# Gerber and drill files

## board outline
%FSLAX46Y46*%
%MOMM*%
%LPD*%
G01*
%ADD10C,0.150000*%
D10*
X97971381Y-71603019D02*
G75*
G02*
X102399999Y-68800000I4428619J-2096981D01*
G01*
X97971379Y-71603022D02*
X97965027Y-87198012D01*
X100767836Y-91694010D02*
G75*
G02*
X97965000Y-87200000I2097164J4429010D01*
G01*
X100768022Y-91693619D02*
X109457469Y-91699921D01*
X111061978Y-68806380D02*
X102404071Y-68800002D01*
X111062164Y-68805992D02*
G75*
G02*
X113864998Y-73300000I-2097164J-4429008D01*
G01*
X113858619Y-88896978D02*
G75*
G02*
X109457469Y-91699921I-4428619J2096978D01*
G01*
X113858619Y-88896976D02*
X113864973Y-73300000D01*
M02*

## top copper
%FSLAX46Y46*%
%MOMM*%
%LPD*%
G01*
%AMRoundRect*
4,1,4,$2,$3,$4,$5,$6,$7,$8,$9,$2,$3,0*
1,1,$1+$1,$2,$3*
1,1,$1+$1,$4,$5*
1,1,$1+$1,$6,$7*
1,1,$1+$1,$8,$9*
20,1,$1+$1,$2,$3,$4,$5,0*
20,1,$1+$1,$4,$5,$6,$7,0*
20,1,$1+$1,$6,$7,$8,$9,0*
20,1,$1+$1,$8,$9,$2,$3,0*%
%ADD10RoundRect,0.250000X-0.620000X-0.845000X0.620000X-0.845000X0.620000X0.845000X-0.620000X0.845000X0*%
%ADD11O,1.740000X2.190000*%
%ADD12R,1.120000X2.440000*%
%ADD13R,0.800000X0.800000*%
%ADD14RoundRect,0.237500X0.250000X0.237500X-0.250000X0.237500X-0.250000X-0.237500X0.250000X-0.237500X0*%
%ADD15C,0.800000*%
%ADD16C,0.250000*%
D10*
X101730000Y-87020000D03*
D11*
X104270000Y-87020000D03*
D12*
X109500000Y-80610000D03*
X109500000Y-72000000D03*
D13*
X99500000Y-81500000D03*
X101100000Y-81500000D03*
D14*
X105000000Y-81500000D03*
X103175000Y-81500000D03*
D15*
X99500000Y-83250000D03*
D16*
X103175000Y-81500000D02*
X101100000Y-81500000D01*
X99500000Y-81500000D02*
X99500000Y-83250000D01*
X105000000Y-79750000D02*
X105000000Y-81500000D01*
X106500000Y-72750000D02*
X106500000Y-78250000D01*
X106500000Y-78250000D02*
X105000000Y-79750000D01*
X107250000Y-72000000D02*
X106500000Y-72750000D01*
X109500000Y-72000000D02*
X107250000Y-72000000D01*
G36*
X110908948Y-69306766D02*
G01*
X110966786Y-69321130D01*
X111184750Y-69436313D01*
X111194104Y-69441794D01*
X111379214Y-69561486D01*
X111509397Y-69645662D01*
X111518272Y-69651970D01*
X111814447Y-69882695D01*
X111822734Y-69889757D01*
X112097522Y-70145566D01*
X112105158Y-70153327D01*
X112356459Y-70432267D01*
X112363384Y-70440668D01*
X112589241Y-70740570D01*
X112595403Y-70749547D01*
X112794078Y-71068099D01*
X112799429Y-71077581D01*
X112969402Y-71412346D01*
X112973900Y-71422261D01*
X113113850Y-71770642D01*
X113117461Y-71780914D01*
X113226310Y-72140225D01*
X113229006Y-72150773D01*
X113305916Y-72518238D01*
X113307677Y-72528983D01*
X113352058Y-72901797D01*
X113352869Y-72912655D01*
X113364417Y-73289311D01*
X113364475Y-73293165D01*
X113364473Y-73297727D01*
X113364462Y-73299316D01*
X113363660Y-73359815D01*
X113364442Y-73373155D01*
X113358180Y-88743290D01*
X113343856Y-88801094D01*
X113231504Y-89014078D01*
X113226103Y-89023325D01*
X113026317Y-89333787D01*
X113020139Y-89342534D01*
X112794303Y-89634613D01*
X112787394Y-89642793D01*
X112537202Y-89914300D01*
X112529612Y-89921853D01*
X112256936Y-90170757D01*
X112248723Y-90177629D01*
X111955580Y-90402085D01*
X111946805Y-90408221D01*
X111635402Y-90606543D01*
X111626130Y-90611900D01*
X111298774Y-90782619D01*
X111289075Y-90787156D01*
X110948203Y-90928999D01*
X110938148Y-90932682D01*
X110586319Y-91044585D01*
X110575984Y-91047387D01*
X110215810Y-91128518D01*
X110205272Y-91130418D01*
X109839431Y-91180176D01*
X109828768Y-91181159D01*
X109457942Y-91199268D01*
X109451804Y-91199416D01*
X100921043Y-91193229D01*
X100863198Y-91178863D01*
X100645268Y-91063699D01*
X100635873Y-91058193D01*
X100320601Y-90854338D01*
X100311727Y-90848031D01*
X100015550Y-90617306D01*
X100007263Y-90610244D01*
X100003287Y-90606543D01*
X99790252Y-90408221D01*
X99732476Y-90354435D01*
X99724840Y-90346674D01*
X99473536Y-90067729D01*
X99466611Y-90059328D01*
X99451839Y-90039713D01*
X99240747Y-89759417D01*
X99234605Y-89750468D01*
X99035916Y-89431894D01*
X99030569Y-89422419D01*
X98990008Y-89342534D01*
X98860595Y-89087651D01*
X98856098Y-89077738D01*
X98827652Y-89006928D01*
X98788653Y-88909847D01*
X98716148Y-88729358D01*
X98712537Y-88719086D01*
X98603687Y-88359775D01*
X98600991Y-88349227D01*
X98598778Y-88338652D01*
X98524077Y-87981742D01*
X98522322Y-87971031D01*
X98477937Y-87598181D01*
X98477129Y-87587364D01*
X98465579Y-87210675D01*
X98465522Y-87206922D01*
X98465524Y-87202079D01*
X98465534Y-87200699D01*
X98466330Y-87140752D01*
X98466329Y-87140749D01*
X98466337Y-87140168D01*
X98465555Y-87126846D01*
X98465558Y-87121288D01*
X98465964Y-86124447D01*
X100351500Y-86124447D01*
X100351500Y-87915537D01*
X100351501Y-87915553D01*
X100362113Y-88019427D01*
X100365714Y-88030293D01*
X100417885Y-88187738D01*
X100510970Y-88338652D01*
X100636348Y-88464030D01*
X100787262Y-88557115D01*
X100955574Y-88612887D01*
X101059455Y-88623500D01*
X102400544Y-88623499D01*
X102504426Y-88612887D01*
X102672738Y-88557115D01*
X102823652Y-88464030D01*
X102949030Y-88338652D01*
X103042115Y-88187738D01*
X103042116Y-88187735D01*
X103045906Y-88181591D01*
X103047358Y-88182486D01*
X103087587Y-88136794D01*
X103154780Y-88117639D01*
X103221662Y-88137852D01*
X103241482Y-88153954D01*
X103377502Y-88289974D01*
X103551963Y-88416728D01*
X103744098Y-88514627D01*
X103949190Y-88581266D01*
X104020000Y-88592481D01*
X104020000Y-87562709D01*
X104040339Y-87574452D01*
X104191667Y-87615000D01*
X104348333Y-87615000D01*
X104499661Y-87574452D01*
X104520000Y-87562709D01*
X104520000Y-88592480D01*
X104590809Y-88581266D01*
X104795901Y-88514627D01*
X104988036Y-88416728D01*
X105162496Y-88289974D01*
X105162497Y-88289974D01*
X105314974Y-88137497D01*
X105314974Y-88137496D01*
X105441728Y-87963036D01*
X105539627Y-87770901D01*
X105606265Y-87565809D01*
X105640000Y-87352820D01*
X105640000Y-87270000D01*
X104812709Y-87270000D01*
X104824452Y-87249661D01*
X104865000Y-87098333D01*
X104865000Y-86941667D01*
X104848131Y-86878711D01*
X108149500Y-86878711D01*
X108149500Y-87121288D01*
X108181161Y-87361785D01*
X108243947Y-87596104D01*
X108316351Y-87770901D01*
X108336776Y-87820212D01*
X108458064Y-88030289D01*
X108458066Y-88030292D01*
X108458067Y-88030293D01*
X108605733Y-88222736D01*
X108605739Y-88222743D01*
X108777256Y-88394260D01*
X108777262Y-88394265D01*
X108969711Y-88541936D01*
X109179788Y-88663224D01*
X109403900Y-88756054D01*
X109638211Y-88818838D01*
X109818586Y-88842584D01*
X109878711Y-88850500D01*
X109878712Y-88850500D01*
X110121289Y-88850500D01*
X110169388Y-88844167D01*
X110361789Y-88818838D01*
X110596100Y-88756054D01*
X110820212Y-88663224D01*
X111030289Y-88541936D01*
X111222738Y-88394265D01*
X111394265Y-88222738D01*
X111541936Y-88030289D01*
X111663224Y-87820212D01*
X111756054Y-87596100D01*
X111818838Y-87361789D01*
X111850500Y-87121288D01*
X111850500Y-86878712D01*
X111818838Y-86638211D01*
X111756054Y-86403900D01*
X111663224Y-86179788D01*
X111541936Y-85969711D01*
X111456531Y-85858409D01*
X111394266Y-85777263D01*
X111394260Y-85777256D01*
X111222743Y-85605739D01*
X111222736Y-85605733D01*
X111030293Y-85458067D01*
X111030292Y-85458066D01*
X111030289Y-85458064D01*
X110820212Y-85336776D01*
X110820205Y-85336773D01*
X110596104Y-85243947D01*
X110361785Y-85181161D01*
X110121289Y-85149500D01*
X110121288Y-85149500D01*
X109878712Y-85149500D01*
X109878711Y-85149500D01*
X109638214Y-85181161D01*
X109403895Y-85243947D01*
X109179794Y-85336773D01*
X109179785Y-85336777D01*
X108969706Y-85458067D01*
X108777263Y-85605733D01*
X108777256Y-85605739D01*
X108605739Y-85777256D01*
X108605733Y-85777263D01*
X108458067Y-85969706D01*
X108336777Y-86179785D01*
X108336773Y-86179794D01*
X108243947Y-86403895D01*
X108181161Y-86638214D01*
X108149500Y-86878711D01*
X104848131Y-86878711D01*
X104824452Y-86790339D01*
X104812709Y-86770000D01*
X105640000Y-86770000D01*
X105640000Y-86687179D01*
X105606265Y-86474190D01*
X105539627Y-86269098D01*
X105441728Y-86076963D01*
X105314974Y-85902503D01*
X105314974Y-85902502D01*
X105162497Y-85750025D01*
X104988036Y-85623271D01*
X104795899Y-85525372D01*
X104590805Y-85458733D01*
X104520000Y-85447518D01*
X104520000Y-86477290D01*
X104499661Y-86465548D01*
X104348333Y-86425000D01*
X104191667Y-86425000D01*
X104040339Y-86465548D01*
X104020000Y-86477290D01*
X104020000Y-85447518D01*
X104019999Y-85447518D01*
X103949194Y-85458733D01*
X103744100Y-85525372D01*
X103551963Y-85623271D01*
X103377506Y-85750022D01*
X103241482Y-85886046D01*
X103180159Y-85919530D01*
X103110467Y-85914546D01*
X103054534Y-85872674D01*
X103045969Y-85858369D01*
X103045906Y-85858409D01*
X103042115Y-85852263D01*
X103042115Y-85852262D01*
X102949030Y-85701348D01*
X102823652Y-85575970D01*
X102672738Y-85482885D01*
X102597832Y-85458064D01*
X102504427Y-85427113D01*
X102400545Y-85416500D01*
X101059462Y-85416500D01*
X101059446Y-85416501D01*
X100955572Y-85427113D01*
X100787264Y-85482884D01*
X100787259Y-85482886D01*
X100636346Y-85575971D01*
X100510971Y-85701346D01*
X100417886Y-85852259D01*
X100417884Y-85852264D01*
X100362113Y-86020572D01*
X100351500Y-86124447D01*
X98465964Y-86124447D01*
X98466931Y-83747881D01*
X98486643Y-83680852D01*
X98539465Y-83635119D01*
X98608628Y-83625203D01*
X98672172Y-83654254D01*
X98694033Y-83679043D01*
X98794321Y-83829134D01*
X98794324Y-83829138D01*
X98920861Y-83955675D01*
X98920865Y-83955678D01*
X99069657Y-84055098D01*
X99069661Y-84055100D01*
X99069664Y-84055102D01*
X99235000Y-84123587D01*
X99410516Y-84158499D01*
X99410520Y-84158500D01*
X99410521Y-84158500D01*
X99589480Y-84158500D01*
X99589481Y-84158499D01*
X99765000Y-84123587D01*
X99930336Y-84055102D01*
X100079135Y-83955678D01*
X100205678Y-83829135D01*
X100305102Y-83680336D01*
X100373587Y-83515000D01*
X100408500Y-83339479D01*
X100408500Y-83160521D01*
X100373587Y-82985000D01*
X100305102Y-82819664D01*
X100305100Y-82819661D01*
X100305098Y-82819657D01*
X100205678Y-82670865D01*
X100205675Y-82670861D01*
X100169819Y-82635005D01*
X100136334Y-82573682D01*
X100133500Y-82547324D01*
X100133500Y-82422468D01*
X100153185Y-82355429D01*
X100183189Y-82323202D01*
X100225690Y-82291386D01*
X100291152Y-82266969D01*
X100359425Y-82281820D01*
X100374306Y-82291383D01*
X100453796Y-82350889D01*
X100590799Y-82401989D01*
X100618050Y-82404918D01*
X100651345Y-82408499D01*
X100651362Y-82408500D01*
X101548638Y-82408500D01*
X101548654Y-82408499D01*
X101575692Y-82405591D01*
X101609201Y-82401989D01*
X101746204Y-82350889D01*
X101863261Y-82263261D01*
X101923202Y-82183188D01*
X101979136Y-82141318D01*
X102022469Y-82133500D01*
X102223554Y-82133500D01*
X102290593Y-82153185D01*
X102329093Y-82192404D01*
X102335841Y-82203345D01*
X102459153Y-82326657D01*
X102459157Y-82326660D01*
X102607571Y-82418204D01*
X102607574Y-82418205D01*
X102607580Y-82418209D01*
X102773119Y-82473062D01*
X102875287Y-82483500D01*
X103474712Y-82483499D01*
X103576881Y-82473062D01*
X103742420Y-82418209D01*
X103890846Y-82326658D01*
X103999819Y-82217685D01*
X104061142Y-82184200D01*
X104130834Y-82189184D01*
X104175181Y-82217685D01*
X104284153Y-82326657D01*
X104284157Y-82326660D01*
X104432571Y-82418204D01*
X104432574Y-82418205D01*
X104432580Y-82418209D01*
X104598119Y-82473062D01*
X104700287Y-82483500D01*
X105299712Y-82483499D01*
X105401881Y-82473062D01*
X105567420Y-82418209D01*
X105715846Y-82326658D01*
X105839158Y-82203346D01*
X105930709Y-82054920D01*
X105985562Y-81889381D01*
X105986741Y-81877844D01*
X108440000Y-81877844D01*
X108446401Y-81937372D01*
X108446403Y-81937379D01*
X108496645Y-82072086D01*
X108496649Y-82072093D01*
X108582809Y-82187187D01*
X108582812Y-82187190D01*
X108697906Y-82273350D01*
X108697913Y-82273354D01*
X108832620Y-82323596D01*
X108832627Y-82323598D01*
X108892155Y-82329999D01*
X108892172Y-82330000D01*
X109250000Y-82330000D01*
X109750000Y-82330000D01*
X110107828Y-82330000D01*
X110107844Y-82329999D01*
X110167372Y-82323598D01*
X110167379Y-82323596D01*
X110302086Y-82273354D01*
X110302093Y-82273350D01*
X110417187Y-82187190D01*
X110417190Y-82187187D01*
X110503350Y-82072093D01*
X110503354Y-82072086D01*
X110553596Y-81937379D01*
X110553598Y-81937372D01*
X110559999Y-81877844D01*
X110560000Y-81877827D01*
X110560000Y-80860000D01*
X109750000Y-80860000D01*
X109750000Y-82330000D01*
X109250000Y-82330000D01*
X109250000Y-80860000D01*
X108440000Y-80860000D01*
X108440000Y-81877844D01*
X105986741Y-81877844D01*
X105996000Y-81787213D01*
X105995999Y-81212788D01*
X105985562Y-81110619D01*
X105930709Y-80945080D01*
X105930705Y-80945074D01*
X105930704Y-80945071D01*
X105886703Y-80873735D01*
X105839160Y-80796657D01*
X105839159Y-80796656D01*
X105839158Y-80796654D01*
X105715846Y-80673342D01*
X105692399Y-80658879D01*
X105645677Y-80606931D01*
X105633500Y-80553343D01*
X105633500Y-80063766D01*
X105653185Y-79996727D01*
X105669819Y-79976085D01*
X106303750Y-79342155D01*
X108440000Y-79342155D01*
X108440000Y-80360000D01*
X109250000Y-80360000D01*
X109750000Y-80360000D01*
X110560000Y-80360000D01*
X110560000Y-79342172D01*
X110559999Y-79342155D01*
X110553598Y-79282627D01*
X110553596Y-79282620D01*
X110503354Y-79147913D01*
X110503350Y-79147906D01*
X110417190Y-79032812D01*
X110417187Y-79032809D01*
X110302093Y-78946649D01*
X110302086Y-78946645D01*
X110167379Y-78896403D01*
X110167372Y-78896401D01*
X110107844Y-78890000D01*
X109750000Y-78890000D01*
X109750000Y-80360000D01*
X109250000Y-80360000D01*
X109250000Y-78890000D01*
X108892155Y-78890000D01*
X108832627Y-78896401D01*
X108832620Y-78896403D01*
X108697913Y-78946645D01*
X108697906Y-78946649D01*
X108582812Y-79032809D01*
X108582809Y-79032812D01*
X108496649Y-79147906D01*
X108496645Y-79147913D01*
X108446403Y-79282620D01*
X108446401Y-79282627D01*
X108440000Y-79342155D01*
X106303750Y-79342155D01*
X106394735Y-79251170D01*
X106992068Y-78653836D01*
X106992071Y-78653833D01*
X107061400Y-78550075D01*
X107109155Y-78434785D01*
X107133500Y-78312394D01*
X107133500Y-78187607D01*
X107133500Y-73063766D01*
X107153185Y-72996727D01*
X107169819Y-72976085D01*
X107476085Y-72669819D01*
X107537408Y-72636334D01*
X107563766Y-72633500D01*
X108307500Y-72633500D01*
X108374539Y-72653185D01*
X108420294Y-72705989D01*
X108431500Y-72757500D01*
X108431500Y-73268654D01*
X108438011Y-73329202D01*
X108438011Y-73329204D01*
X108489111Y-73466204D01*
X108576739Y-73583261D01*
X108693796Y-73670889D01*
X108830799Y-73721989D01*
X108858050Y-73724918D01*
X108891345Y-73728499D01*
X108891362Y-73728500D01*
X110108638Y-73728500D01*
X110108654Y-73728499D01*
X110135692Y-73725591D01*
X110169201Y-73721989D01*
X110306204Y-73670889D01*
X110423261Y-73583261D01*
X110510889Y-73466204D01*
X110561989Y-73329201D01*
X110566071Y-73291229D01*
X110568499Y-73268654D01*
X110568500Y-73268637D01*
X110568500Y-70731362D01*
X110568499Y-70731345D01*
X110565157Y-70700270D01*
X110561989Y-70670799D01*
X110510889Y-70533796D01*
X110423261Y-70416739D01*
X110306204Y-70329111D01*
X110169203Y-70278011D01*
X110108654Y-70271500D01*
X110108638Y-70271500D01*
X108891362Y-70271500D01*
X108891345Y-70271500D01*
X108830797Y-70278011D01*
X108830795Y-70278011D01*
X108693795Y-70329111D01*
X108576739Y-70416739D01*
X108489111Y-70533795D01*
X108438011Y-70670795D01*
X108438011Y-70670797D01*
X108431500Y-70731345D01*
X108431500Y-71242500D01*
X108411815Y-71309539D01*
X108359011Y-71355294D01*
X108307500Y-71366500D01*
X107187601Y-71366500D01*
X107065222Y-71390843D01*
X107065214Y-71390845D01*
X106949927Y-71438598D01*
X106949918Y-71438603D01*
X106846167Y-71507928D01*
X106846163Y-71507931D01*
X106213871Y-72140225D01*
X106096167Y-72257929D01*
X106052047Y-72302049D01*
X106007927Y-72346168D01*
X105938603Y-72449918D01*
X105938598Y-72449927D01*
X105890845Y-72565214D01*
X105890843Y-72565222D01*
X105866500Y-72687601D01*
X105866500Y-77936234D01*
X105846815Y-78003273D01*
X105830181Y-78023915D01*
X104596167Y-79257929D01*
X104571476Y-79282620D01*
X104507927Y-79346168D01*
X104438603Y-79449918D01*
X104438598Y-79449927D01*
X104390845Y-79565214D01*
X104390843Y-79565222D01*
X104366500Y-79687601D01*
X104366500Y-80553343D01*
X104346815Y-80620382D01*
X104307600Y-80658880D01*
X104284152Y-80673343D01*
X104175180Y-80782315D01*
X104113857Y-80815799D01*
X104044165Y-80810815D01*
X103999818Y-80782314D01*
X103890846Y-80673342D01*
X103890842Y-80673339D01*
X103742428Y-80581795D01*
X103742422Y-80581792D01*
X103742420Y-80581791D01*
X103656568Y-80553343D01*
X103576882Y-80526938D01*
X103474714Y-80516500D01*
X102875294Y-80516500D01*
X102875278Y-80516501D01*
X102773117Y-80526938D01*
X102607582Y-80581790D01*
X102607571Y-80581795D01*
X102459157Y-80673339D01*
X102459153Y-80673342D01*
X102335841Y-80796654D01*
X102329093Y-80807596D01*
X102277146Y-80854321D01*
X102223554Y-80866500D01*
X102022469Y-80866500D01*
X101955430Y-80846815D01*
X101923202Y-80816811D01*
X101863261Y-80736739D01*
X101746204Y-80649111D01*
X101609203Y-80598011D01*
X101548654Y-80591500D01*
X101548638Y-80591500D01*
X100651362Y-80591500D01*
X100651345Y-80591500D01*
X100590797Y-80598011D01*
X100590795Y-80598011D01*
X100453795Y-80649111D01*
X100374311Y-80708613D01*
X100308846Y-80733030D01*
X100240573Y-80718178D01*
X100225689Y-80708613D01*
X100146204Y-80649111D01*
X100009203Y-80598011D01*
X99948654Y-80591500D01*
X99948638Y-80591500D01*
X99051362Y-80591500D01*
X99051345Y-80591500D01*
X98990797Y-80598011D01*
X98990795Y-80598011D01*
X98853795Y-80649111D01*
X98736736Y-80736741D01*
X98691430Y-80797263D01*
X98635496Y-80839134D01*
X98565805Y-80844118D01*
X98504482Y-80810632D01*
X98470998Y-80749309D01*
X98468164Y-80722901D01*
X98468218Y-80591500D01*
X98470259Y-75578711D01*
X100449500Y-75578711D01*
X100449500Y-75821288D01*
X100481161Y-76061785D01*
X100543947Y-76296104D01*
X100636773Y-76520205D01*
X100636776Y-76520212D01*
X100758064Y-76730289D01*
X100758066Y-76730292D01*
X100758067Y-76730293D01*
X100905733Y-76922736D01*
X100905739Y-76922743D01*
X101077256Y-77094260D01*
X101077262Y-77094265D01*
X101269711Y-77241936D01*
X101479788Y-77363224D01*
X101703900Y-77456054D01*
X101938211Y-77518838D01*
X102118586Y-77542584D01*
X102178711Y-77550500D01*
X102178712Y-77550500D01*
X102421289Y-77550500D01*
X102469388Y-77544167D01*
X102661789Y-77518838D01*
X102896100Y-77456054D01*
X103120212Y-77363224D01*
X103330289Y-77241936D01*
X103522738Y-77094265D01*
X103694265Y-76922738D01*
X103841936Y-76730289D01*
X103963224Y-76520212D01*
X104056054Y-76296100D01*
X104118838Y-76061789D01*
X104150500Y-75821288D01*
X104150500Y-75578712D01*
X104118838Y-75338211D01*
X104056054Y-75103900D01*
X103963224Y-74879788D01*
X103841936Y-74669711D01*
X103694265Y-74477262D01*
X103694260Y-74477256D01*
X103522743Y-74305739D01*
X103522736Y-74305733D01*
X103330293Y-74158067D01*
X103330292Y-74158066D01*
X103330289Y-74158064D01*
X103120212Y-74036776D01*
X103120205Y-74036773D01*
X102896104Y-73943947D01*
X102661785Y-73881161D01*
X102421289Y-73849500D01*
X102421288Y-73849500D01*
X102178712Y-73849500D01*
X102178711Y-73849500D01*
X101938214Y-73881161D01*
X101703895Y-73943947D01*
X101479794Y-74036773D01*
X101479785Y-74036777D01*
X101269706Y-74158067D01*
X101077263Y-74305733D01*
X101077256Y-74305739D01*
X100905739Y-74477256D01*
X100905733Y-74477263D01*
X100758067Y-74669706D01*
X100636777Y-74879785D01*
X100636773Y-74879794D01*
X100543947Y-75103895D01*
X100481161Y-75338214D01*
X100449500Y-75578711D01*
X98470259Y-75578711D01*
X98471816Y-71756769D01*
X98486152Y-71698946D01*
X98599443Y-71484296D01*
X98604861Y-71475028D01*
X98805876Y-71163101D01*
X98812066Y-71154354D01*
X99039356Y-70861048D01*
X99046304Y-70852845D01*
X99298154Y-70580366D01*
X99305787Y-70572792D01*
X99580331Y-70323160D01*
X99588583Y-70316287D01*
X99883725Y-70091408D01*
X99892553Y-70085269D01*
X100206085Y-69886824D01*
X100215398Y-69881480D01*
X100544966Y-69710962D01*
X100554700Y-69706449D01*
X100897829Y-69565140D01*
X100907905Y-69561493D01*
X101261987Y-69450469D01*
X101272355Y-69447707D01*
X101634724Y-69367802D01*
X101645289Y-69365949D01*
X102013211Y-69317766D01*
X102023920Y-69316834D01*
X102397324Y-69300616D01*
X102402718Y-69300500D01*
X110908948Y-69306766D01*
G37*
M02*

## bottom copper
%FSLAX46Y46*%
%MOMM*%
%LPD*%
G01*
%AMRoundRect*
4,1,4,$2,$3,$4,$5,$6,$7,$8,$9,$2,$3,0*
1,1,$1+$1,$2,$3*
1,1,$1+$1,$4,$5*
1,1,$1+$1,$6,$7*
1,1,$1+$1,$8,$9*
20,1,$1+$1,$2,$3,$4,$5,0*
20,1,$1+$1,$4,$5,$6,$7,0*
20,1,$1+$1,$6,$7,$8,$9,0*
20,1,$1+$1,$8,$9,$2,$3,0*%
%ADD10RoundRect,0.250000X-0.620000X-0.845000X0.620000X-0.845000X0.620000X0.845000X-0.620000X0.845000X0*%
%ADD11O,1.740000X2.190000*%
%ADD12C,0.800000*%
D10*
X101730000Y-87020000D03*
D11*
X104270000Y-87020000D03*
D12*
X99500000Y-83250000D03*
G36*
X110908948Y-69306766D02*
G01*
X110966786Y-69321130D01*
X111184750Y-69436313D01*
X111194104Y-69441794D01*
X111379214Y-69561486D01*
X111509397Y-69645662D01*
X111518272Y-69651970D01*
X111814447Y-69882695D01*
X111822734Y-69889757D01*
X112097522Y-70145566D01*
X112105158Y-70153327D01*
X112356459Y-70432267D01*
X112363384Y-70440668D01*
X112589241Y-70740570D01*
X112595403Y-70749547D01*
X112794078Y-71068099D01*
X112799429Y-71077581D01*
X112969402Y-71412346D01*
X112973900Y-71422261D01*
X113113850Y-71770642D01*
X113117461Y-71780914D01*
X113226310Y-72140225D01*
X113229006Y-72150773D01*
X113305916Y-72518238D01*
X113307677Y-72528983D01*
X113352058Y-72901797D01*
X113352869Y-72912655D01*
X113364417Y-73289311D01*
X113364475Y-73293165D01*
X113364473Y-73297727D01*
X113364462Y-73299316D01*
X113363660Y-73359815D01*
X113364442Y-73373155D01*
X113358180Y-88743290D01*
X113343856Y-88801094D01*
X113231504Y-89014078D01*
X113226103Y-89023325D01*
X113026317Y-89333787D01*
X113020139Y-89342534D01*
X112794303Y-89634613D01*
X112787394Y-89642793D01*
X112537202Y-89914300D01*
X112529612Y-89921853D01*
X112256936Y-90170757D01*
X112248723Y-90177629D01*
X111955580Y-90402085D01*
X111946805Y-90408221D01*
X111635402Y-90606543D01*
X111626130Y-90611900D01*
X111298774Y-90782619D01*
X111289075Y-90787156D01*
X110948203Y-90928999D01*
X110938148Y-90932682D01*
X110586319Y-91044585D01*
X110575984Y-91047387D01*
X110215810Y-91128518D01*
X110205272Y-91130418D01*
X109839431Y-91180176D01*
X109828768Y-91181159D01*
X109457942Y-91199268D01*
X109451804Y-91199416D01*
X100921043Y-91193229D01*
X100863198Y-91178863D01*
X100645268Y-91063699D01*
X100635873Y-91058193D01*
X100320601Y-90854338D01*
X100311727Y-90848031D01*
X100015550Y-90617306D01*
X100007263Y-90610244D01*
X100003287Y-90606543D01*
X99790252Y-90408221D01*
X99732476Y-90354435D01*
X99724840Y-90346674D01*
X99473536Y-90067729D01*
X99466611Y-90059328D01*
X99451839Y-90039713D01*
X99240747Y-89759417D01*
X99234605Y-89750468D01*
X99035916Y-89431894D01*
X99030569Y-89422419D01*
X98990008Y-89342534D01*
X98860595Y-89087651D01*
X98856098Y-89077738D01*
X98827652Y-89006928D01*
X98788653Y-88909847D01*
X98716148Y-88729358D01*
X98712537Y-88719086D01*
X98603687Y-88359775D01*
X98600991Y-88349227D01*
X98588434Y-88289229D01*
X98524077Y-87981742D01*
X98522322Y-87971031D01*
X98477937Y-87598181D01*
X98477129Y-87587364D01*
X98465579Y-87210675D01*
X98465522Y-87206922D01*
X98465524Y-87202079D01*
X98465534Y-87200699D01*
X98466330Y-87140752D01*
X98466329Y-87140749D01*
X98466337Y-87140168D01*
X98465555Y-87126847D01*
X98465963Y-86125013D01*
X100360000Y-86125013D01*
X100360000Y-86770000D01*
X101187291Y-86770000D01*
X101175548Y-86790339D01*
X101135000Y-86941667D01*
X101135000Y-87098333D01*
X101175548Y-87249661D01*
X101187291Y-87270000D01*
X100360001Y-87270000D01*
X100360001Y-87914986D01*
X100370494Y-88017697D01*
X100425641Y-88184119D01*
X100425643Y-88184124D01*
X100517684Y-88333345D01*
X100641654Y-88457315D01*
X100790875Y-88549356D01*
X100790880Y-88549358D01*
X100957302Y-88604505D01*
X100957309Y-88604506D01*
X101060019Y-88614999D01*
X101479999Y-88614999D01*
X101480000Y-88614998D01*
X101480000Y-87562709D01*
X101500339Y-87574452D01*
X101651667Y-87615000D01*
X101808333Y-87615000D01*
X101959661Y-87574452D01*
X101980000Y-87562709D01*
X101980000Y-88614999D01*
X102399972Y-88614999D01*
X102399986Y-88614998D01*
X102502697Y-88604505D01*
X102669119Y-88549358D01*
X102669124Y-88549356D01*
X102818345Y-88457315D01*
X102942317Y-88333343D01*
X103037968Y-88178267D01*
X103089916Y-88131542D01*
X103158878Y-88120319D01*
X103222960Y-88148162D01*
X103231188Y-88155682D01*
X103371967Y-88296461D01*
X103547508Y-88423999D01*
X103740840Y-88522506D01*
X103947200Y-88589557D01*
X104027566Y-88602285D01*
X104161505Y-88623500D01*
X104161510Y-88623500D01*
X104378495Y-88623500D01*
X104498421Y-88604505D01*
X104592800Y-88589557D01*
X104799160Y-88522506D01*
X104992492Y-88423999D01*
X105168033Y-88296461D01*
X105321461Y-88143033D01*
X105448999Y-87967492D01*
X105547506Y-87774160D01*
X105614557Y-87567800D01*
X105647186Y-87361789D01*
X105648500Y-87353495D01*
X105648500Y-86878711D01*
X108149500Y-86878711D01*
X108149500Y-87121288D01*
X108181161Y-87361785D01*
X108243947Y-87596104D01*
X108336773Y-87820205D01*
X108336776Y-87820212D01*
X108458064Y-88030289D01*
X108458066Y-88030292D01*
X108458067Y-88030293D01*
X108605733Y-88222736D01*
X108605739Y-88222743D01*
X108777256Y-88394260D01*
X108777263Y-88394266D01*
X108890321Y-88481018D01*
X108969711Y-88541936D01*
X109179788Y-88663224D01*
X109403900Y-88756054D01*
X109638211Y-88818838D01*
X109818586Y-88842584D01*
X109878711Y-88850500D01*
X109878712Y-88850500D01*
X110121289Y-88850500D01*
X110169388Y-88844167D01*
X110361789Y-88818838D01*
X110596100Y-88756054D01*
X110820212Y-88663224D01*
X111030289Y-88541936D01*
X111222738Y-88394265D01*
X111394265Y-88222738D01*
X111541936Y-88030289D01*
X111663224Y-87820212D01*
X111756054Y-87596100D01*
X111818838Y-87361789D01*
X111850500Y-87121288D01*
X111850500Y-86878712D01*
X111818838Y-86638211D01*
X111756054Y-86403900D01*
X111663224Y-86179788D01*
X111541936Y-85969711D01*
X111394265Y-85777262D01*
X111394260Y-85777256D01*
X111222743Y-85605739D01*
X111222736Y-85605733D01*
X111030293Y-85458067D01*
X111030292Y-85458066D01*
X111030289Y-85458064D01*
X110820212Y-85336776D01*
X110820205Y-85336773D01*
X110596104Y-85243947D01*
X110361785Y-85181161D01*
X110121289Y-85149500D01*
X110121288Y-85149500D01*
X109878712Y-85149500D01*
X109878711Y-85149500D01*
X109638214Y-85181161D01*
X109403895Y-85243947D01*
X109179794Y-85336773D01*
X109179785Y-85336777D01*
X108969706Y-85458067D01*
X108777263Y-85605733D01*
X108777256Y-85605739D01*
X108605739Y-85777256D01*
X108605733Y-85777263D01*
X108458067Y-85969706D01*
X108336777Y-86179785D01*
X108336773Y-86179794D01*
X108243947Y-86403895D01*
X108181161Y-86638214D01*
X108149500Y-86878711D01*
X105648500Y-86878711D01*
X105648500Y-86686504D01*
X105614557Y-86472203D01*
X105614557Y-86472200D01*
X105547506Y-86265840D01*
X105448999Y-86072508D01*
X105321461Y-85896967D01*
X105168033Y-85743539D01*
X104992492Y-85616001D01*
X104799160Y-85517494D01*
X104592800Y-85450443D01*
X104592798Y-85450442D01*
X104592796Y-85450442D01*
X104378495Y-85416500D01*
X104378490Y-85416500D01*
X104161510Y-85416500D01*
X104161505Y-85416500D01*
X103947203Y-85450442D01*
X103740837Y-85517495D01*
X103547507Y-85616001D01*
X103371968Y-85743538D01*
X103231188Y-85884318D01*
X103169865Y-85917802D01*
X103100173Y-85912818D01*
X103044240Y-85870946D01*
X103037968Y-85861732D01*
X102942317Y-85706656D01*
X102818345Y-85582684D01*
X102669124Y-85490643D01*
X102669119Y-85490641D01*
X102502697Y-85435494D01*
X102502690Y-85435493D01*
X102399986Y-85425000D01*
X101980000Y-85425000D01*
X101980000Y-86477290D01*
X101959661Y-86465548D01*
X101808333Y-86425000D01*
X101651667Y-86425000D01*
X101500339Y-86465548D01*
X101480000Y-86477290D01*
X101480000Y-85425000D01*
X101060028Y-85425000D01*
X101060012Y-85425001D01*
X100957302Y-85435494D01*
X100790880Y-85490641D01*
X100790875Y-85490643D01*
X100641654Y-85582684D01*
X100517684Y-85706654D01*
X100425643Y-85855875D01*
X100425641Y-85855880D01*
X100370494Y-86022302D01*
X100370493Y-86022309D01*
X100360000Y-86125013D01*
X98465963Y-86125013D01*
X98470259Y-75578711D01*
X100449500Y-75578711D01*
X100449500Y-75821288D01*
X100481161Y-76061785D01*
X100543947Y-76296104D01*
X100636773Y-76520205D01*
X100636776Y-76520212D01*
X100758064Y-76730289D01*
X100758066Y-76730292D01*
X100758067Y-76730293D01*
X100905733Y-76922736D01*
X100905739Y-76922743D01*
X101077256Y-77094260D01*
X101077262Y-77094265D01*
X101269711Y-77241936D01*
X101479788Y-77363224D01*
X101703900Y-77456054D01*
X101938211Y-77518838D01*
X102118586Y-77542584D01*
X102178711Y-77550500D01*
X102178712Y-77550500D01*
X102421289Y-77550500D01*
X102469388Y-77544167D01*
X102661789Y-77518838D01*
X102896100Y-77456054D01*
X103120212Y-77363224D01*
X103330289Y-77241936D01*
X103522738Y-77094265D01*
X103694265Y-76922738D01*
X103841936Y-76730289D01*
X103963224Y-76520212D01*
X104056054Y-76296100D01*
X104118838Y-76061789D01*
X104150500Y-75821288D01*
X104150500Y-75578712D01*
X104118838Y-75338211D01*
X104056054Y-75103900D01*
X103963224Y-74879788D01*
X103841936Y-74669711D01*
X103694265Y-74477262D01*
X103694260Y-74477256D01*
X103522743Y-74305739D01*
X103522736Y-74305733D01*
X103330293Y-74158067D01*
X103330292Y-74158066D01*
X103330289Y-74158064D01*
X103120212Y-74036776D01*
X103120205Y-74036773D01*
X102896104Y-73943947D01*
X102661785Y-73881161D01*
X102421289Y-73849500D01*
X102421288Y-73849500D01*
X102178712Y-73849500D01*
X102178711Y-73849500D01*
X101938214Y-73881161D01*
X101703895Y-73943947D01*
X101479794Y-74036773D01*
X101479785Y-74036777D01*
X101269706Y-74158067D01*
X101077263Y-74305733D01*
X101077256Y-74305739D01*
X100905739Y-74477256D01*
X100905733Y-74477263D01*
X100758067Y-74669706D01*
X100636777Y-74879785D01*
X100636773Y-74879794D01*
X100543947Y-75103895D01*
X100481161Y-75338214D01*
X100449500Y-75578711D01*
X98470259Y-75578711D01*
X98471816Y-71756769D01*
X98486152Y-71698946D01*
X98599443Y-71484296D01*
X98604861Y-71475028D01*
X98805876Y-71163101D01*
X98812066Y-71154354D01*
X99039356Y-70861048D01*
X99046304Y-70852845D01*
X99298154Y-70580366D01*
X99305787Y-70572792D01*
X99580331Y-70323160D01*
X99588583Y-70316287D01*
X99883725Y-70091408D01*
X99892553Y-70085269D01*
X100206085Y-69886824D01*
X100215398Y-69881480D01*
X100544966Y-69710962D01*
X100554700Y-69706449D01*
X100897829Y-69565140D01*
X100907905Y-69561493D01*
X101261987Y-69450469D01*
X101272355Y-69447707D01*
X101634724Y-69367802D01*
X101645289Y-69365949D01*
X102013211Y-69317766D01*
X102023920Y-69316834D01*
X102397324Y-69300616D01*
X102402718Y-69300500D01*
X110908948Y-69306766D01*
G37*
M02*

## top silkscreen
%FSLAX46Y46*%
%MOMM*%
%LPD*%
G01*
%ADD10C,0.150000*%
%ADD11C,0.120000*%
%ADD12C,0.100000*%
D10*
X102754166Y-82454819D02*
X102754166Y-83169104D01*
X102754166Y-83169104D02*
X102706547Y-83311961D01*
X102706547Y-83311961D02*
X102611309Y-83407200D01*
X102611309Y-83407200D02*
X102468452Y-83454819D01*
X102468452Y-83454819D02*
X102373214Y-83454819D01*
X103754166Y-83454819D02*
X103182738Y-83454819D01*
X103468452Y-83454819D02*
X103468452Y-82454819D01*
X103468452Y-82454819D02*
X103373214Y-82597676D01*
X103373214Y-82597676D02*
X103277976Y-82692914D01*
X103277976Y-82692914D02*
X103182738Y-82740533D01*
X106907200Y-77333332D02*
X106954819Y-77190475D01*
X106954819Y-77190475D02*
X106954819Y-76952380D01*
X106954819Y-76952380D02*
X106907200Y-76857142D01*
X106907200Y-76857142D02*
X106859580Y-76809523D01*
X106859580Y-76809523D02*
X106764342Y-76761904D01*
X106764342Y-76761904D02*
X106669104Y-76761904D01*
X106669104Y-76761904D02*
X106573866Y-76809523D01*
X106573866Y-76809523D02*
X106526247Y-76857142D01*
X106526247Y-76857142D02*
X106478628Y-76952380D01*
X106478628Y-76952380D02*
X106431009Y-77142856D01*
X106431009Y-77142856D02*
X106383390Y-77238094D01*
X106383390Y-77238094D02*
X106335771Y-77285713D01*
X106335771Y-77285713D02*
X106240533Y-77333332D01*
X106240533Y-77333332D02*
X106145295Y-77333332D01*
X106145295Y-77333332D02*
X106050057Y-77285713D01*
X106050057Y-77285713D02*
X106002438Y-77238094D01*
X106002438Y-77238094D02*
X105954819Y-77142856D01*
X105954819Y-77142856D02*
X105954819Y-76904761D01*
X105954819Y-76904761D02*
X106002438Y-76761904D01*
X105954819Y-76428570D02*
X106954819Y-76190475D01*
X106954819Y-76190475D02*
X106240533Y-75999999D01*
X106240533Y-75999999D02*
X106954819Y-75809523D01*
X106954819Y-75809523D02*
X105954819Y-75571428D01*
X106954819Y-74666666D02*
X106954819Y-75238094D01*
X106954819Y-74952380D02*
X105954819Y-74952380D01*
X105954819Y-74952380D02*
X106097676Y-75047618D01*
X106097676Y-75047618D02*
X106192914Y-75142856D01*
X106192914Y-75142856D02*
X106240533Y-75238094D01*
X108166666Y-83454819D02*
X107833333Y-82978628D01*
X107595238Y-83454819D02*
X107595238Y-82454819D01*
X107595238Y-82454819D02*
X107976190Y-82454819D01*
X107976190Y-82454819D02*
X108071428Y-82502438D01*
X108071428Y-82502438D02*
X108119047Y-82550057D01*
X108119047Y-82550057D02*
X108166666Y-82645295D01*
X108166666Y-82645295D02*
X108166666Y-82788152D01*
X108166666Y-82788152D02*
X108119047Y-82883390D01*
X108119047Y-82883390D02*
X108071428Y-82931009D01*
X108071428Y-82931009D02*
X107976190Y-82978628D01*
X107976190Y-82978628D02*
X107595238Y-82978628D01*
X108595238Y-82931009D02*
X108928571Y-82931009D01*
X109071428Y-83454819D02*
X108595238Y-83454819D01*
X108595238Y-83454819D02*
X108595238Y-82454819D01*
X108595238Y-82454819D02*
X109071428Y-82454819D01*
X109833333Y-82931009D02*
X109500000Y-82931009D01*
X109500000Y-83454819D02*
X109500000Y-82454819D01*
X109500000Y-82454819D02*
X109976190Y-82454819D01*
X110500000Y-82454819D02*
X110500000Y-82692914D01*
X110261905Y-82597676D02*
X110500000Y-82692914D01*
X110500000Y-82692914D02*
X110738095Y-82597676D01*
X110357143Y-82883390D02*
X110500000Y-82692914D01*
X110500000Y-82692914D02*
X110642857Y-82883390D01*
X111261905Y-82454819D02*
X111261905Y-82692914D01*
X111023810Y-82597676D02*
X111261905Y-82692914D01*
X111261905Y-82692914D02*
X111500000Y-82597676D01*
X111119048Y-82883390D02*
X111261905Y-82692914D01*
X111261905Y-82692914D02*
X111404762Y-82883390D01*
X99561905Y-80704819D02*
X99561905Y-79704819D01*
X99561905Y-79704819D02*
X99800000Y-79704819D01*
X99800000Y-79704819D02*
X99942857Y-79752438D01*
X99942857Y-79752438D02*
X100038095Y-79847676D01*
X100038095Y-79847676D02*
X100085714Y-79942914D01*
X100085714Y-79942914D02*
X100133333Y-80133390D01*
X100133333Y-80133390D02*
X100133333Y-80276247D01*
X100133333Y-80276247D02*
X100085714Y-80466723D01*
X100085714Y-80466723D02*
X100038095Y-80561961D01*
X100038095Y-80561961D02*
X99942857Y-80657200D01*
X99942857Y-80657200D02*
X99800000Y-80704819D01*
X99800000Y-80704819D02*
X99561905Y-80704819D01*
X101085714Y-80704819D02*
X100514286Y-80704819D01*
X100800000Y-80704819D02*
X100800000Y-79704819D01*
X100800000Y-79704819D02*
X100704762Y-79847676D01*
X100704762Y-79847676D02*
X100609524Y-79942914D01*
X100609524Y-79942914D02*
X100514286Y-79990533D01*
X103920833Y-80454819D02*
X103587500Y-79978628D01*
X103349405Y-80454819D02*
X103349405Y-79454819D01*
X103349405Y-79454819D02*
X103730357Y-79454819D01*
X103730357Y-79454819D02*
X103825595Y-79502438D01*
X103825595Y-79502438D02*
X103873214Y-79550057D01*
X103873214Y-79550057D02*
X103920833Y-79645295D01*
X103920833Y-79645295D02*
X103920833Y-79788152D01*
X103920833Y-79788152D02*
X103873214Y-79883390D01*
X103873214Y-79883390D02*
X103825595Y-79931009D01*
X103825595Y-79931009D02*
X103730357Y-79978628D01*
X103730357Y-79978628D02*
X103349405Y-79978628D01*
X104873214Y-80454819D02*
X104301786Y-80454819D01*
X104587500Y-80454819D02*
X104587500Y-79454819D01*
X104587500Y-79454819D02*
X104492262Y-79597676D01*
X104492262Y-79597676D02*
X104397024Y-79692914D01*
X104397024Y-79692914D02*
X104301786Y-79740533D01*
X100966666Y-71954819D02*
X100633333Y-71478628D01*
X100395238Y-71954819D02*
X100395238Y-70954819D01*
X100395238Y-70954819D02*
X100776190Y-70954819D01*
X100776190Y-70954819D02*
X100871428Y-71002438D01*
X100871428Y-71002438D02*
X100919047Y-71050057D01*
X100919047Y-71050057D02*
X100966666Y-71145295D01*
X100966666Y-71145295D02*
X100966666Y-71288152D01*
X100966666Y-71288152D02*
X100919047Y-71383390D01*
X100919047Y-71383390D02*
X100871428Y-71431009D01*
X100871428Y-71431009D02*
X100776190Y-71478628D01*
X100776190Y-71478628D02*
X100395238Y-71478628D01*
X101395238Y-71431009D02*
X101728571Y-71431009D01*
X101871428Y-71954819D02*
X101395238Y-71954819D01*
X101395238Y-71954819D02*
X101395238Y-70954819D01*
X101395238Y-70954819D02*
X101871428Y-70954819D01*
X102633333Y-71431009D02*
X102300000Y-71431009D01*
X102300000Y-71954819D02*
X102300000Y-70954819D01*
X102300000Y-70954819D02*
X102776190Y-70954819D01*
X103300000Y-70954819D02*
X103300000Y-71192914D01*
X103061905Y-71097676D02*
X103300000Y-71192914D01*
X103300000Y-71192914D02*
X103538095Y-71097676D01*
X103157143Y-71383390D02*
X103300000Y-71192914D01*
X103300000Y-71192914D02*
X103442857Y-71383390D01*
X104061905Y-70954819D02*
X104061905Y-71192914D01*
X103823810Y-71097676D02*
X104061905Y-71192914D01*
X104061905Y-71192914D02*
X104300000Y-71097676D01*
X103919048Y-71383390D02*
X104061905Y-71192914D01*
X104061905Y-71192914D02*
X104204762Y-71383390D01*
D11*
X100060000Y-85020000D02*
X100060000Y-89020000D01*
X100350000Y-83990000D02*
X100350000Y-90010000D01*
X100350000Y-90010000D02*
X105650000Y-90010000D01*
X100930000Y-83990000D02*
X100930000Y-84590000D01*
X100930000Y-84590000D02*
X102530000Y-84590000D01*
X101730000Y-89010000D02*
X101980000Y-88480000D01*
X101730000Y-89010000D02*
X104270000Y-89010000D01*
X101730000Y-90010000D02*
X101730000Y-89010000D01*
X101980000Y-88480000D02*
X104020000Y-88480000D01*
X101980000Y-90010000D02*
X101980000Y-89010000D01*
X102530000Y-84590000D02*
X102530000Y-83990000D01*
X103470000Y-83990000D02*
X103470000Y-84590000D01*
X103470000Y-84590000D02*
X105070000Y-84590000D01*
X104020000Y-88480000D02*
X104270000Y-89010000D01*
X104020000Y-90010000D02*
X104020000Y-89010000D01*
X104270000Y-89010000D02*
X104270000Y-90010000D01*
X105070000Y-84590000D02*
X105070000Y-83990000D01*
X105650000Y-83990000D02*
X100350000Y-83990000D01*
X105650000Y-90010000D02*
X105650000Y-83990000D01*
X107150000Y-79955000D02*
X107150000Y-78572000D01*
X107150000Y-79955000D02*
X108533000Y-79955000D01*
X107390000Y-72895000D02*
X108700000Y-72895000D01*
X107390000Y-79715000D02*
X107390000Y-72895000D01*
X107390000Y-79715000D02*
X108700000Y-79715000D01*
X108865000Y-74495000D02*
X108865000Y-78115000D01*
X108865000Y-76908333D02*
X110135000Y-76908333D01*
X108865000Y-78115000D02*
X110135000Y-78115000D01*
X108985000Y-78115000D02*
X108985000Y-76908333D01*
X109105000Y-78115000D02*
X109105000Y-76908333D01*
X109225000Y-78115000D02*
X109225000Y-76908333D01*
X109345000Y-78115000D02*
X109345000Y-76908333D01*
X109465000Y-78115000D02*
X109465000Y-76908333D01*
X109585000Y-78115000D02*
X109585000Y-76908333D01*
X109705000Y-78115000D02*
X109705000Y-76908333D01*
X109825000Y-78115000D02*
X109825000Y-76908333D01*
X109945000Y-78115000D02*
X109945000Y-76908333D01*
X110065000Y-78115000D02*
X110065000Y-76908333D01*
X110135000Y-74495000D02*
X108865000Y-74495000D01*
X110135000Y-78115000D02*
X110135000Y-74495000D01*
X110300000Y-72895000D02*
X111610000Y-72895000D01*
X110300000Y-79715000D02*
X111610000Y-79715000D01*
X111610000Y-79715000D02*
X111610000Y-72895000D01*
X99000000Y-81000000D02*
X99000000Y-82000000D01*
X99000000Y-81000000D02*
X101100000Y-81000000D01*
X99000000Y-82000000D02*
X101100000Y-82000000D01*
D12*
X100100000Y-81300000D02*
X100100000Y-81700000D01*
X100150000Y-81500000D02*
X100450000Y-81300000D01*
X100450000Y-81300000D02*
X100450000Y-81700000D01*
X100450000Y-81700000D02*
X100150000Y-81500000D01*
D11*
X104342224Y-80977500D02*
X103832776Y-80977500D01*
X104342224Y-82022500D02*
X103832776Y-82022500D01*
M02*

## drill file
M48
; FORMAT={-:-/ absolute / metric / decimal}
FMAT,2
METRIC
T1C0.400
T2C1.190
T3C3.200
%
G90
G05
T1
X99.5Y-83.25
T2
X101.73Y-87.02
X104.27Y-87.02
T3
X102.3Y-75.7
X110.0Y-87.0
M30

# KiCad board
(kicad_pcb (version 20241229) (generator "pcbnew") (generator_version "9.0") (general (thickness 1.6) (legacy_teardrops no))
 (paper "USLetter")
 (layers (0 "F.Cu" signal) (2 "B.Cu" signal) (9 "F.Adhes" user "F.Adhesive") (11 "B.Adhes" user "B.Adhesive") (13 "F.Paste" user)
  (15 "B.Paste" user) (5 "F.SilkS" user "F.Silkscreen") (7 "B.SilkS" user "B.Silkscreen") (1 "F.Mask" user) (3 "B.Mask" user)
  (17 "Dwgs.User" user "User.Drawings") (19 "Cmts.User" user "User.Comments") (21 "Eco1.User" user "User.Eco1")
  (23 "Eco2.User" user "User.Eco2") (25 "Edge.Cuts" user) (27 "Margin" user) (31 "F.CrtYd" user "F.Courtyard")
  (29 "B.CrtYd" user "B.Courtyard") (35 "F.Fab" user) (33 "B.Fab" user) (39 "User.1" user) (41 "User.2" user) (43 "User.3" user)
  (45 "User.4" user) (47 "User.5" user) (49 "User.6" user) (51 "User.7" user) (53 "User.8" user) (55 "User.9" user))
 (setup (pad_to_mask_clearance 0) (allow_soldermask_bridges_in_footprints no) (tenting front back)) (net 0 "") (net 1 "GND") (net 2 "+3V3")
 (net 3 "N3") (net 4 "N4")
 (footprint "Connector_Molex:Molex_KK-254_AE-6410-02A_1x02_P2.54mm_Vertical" (layer "F.Cu") (at 101.73 87.02)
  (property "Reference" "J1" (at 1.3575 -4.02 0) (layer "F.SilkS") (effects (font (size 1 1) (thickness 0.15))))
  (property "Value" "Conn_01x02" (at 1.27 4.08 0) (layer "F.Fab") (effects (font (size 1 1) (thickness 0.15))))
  (fp_line (start -1.67 -2) (end -1.67 2) (stroke (width 0.12) (type solid)) (layer "F.SilkS"))
  (fp_line (start -1.38 -3.03) (end -1.38 2.99) (stroke (width 0.12) (type solid)) (layer "F.SilkS"))
  (fp_line (start -1.38 2.99) (end 3.92 2.99) (stroke (width 0.12) (type solid)) (layer "F.SilkS"))
  (fp_line (start -0.8 -3.03) (end -0.8 -2.43) (stroke (width 0.12) (type solid)) (layer "F.SilkS"))
  (fp_line (start -0.8 -2.43) (end 0.8 -2.43) (stroke (width 0.12) (type solid)) (layer "F.SilkS"))
  (fp_line (start 0 1.99) (end 0.25 1.46) (stroke (width 0.12) (type solid)) (layer "F.SilkS"))
  (fp_line (start 0 1.99) (end 2.54 1.99) (stroke (width 0.12) (type solid)) (layer "F.SilkS"))
  (fp_line (start 0 2.99) (end 0 1.99) (stroke (width 0.12) (type solid)) (layer "F.SilkS"))
  (fp_line (start 0.25 1.46) (end 2.29 1.46) (stroke (width 0.12) (type solid)) (layer "F.SilkS"))
  (fp_line (start 0.25 2.99) (end 0.25 1.99) (stroke (width 0.12) (type solid)) (layer "F.SilkS"))
  (fp_line (start 0.8 -2.43) (end 0.8 -3.03) (stroke (width 0.12) (type solid)) (layer "F.SilkS"))
  (fp_line (start 1.74 -3.03) (end 1.74 -2.43) (stroke (width 0.12) (type solid)) (layer "F.SilkS"))
  (fp_line (start 1.74 -2.43) (end 3.34 -2.43) (stroke (width 0.12) (type solid)) (layer "F.SilkS"))
  (fp_line (start 2.29 1.46) (end 2.54 1.99) (stroke (width 0.12) (type solid)) (layer "F.SilkS"))
  (fp_line (start 2.29 2.99) (end 2.29 1.99) (stroke (width 0.12) (type solid)) (layer "F.SilkS"))
  (fp_line (start 2.54 1.99) (end 2.54 2.99) (stroke (width 0.12) (type solid)) (layer "F.SilkS"))
  (fp_line (start 3.34 -2.43) (end 3.34 -3.03) (stroke (width 0.12) (type solid)) (layer "F.SilkS"))
  (fp_line (start 3.92 -3.03) (end -1.38 -3.03) (stroke (width 0.12) (type solid)) (layer "F.SilkS"))
  (fp_line (start 3.92 2.99) (end 3.92 -3.03) (stroke (width 0.12) (type solid)) (layer "F.SilkS"))
  (pad "1" thru_hole roundrect (at 0 0) (size 1.74 2.19) (drill 1.19) (layers "*.Cu" "*.Mask") (remove_unused_layers no)
   (roundrect_rratio 0.143678) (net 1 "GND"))
  (pad "2" thru_hole oval (at 2.54 0) (size 1.74 2.19) (drill 1.19) (layers "*.Cu" "*.Mask") (remove_unused_layers no) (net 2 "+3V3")))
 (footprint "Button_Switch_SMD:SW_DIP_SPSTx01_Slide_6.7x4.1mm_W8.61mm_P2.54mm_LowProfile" (layer "F.Cu") (at 109.5 76.305 90)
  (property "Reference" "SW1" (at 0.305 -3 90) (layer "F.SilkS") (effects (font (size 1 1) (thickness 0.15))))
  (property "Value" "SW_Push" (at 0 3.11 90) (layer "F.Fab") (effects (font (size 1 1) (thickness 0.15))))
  (fp_line (start -3.65 -2.35) (end -2.267 -2.35) (stroke (width 0.12) (type solid)) (layer "F.SilkS"))
  (fp_line (start -3.65 -2.35) (end -3.65 -0.967) (stroke (width 0.12) (type solid)) (layer "F.SilkS"))
  (fp_line (start 3.41 -2.11) (end 3.41 -0.8) (stroke (width 0.12) (type solid)) (layer "F.SilkS"))
  (fp_line (start -3.41 -2.11) (end 3.41 -2.11) (stroke (width 0.12) (type solid)) (layer "F.SilkS"))
  (fp_line (start -3.41 -2.11) (end -3.41 -0.8) (stroke (width 0.12) (type solid)) (layer "F.SilkS"))
  (fp_line (start 1.81 -0.635) (end -1.81 -0.635) (stroke (width 0.12) (type solid)) (layer "F.SilkS"))
  (fp_line (start -0.603333 -0.635) (end -0.603333 0.635) (stroke (width 0.12) (type solid)) (layer "F.SilkS"))
  (fp_line (start -1.81 -0.635) (end -1.81 0.635) (stroke (width 0.12) (type solid)) (layer "F.SilkS"))
  (fp_line (start -1.81 -0.515) (end -0.603333 -0.515) (stroke (width 0.12) (type solid)) (layer "F.SilkS"))
  (fp_line (start -1.81 -0.395) (end -0.603333 -0.395) (stroke (width 0.12) (type solid)) (layer "F.SilkS"))
  (fp_line (start -1.81 -0.275) (end -0.603333 -0.275) (stroke (width 0.12) (type solid)) (layer "F.SilkS"))
  (fp_line (start -1.81 -0.155) (end -0.603333 -0.155) (stroke (width 0.12) (type solid)) (layer "F.SilkS"))
  (fp_line (start -1.81 -0.035) (end -0.603333 -0.035) (stroke (width 0.12) (type solid)) (layer "F.SilkS"))
  (fp_line (start -1.81 0.085) (end -0.603333 0.085) (stroke (width 0.12) (type solid)) (layer "F.SilkS"))
  (fp_line (start -1.81 0.205) (end -0.603333 0.205) (stroke (width 0.12) (type solid)) (layer "F.SilkS"))
  (fp_line (start -1.81 0.325) (end -0.603333 0.325) (stroke (width 0.12) (type solid)) (layer "F.SilkS"))
  (fp_line (start -1.81 0.445) (end -0.603333 0.445) (stroke (width 0.12) (type solid)) (layer "F.SilkS"))
  (fp_line (start -1.81 0.565) (end -0.603333 0.565) (stroke (width 0.12) (type solid)) (layer "F.SilkS"))
  (fp_line (start 1.81 0.635) (end 1.81 -0.635) (stroke (width 0.12) (type solid)) (layer "F.SilkS"))
  (fp_line (start -1.81 0.635) (end 1.81 0.635) (stroke (width 0.12) (type solid)) (layer "F.SilkS"))
  (fp_line (start 3.41 0.8) (end 3.41 2.11) (stroke (width 0.12) (type solid)) (layer "F.SilkS"))
  (fp_line (start -3.41 0.8) (end -3.41 2.11) (stroke (width 0.12) (type solid)) (layer "F.SilkS"))
  (fp_line (start -3.41 2.11) (end 3.41 2.11) (stroke (width 0.12) (type solid)) (layer "F.SilkS"))
  (pad "1" smd rect (at -4.305 0 90) (size 2.44 1.12) (layers "F.Cu" "F.Mask" "F.Paste") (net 2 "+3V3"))
  (pad "2" smd rect (at 4.305 0 90) (size 2.44 1.12) (layers "F.Cu" "F.Mask" "F.Paste") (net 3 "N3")))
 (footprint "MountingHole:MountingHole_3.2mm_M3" (layer "F.Cu") (at 110 87)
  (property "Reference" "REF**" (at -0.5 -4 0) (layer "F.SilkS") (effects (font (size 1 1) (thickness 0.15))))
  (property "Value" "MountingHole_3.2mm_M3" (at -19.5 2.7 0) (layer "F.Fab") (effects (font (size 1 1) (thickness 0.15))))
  (pad "" np_thru_hole circle (at 0 0) (size 3.2 3.2) (drill 3.2) (layers "*.Cu" "*.Mask")))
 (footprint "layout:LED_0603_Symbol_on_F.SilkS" (layer "F.Cu") (at 100.3 81.5)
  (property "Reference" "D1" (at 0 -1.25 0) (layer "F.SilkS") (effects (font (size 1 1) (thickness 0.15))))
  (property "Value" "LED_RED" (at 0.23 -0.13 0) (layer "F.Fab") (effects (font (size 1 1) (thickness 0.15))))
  (fp_line (start -1.3 -0.5) (end -1.3 0.5) (stroke (width 0.12) (type solid)) (layer "F.SilkS"))
  (fp_line (start -1.3 -0.5) (end 0.8 -0.5) (stroke (width 0.12) (type solid)) (layer "F.SilkS"))
  (fp_line (start -1.3 0.5) (end 0.8 0.5) (stroke (width 0.12) (type solid)) (layer "F.SilkS"))
  (fp_line (start -0.2 -0.2) (end -0.2 0.2) (stroke (width 0.1) (type solid)) (layer "F.SilkS"))
  (fp_line (start -0.15 0) (end 0.15 -0.2) (stroke (width 0.1) (type solid)) (layer "F.SilkS"))
  (fp_line (start 0.15 -0.2) (end 0.15 0.2) (stroke (width 0.1) (type solid)) (layer "F.SilkS"))
  (fp_line (start 0.15 0.2) (end -0.15 0) (stroke (width 0.1) (type solid)) (layer "F.SilkS"))
  (pad "1" smd rect (at -0.8 0 180) (size 0.8 0.8) (layers "F.Cu" "F.Mask" "F.Paste") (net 1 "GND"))
  (pad "2" smd rect (at 0.8 0 180) (size 0.8 0.8) (layers "F.Cu" "F.Mask" "F.Paste") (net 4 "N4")))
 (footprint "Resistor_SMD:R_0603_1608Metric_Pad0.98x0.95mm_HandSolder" (layer "F.Cu") (at 104.0875 81.5 180)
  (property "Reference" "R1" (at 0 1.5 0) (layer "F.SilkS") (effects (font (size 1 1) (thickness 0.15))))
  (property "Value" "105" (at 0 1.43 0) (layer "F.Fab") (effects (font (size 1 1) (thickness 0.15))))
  (fp_line (start -0.254724 0.5225) (end 0.254724 0.5225) (stroke (width 0.12) (type solid)) (layer "F.SilkS"))
  (fp_line (start -0.254724 -0.5225) (end 0.254724 -0.5225) (stroke (width 0.12) (type solid)) (layer "F.SilkS"))
  (pad "1" smd roundrect (at -0.9125 0 180) (size 0.975 0.95) (layers "F.Cu" "F.Mask" "F.Paste") (roundrect_rratio 0.25) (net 3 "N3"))
  (pad "2" smd roundrect (at 0.9125 0 180) (size 0.975 0.95) (layers "F.Cu" "F.Mask" "F.Paste") (roundrect_rratio 0.25) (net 4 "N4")))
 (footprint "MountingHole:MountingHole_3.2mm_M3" (layer "F.Cu") (at 102.3 75.7)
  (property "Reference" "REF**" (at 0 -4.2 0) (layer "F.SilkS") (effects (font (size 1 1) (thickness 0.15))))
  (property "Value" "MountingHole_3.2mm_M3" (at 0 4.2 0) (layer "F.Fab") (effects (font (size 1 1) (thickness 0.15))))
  (pad "" np_thru_hole circle (at 0 0) (size 3.2 3.2) (drill 3.2) (layers "*.Cu" "*.Mask")))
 (gr_arc (start 97.971381 71.603019) (mid 99.779428 69.559638) (end 102.399999 68.8) (stroke (width 0.15) (type solid)) (layer "Edge.Cuts"))
 (gr_line (start 97.971379 71.603022) (end 97.965027 87.198012) (stroke (width 0.15) (type solid)) (layer "Edge.Cuts"))
 (gr_arc (start 100.767836 91.69401) (mid 98.706983 89.858283) (end 97.965 87.2) (stroke (width 0.15) (type solid)) (layer "Edge.Cuts"))
 (gr_line (start 100.768022 91.693619) (end 109.457469 91.699921) (stroke (width 0.15) (type solid)) (layer "Edge.Cuts"))
 (gr_line (start 111.061978 68.80638) (end 102.404071 68.800002) (stroke (width 0.15) (type solid)) (layer "Edge.Cuts"))
 (gr_arc (start 111.062164 68.805992) (mid 113.123016 70.641718) (end 113.864998 73.3) (stroke (width 0.15) (type solid))
  (layer "Edge.Cuts"))
 (gr_arc (start 113.858619 88.896978) (mid 112.062167 90.932999) (end 109.457469 91.699921) (stroke (width 0.15) (type solid))
  (layer "Edge.Cuts"))
 (gr_line (start 113.858619 88.896976) (end 113.864973 73.3) (stroke (width 0.15) (type solid)) (layer "Edge.Cuts"))
 (segment (start 103.175 81.5) (end 101.1 81.5) (width 0.25) (layer "F.Cu") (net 4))
 (segment (start 99.5 81.5) (end 99.5 83.25) (width 0.25) (layer "F.Cu") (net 1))
 (via (at 99.5 83.25) (size 0.8) (drill 0.4) (layers "F.Cu" "B.Cu") (free yes) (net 1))
 (segment (start 105 79.75) (end 105 81.5) (width 0.25) (layer "F.Cu") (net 3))
 (segment (start 106.5 72.75) (end 106.5 78.25) (width 0.25) (layer "F.Cu") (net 3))
 (segment (start 106.5 78.25) (end 105 79.75) (width 0.25) (layer "F.Cu") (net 3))
 (segment (start 107.25 72) (end 106.5 72.75) (width 0.25) (layer "F.Cu") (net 3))
 (segment (start 109.5 72) (end 107.25 72) (width 0.25) (layer "F.Cu") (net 3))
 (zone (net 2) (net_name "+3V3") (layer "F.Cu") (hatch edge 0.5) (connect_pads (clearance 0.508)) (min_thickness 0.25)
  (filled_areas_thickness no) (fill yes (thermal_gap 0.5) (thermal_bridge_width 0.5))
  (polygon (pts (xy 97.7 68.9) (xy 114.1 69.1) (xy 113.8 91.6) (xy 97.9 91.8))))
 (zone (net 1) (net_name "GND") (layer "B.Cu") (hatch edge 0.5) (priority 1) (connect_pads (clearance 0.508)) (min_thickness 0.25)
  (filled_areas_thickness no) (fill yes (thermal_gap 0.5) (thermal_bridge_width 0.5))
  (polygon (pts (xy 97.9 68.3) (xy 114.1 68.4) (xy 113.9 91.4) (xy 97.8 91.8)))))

